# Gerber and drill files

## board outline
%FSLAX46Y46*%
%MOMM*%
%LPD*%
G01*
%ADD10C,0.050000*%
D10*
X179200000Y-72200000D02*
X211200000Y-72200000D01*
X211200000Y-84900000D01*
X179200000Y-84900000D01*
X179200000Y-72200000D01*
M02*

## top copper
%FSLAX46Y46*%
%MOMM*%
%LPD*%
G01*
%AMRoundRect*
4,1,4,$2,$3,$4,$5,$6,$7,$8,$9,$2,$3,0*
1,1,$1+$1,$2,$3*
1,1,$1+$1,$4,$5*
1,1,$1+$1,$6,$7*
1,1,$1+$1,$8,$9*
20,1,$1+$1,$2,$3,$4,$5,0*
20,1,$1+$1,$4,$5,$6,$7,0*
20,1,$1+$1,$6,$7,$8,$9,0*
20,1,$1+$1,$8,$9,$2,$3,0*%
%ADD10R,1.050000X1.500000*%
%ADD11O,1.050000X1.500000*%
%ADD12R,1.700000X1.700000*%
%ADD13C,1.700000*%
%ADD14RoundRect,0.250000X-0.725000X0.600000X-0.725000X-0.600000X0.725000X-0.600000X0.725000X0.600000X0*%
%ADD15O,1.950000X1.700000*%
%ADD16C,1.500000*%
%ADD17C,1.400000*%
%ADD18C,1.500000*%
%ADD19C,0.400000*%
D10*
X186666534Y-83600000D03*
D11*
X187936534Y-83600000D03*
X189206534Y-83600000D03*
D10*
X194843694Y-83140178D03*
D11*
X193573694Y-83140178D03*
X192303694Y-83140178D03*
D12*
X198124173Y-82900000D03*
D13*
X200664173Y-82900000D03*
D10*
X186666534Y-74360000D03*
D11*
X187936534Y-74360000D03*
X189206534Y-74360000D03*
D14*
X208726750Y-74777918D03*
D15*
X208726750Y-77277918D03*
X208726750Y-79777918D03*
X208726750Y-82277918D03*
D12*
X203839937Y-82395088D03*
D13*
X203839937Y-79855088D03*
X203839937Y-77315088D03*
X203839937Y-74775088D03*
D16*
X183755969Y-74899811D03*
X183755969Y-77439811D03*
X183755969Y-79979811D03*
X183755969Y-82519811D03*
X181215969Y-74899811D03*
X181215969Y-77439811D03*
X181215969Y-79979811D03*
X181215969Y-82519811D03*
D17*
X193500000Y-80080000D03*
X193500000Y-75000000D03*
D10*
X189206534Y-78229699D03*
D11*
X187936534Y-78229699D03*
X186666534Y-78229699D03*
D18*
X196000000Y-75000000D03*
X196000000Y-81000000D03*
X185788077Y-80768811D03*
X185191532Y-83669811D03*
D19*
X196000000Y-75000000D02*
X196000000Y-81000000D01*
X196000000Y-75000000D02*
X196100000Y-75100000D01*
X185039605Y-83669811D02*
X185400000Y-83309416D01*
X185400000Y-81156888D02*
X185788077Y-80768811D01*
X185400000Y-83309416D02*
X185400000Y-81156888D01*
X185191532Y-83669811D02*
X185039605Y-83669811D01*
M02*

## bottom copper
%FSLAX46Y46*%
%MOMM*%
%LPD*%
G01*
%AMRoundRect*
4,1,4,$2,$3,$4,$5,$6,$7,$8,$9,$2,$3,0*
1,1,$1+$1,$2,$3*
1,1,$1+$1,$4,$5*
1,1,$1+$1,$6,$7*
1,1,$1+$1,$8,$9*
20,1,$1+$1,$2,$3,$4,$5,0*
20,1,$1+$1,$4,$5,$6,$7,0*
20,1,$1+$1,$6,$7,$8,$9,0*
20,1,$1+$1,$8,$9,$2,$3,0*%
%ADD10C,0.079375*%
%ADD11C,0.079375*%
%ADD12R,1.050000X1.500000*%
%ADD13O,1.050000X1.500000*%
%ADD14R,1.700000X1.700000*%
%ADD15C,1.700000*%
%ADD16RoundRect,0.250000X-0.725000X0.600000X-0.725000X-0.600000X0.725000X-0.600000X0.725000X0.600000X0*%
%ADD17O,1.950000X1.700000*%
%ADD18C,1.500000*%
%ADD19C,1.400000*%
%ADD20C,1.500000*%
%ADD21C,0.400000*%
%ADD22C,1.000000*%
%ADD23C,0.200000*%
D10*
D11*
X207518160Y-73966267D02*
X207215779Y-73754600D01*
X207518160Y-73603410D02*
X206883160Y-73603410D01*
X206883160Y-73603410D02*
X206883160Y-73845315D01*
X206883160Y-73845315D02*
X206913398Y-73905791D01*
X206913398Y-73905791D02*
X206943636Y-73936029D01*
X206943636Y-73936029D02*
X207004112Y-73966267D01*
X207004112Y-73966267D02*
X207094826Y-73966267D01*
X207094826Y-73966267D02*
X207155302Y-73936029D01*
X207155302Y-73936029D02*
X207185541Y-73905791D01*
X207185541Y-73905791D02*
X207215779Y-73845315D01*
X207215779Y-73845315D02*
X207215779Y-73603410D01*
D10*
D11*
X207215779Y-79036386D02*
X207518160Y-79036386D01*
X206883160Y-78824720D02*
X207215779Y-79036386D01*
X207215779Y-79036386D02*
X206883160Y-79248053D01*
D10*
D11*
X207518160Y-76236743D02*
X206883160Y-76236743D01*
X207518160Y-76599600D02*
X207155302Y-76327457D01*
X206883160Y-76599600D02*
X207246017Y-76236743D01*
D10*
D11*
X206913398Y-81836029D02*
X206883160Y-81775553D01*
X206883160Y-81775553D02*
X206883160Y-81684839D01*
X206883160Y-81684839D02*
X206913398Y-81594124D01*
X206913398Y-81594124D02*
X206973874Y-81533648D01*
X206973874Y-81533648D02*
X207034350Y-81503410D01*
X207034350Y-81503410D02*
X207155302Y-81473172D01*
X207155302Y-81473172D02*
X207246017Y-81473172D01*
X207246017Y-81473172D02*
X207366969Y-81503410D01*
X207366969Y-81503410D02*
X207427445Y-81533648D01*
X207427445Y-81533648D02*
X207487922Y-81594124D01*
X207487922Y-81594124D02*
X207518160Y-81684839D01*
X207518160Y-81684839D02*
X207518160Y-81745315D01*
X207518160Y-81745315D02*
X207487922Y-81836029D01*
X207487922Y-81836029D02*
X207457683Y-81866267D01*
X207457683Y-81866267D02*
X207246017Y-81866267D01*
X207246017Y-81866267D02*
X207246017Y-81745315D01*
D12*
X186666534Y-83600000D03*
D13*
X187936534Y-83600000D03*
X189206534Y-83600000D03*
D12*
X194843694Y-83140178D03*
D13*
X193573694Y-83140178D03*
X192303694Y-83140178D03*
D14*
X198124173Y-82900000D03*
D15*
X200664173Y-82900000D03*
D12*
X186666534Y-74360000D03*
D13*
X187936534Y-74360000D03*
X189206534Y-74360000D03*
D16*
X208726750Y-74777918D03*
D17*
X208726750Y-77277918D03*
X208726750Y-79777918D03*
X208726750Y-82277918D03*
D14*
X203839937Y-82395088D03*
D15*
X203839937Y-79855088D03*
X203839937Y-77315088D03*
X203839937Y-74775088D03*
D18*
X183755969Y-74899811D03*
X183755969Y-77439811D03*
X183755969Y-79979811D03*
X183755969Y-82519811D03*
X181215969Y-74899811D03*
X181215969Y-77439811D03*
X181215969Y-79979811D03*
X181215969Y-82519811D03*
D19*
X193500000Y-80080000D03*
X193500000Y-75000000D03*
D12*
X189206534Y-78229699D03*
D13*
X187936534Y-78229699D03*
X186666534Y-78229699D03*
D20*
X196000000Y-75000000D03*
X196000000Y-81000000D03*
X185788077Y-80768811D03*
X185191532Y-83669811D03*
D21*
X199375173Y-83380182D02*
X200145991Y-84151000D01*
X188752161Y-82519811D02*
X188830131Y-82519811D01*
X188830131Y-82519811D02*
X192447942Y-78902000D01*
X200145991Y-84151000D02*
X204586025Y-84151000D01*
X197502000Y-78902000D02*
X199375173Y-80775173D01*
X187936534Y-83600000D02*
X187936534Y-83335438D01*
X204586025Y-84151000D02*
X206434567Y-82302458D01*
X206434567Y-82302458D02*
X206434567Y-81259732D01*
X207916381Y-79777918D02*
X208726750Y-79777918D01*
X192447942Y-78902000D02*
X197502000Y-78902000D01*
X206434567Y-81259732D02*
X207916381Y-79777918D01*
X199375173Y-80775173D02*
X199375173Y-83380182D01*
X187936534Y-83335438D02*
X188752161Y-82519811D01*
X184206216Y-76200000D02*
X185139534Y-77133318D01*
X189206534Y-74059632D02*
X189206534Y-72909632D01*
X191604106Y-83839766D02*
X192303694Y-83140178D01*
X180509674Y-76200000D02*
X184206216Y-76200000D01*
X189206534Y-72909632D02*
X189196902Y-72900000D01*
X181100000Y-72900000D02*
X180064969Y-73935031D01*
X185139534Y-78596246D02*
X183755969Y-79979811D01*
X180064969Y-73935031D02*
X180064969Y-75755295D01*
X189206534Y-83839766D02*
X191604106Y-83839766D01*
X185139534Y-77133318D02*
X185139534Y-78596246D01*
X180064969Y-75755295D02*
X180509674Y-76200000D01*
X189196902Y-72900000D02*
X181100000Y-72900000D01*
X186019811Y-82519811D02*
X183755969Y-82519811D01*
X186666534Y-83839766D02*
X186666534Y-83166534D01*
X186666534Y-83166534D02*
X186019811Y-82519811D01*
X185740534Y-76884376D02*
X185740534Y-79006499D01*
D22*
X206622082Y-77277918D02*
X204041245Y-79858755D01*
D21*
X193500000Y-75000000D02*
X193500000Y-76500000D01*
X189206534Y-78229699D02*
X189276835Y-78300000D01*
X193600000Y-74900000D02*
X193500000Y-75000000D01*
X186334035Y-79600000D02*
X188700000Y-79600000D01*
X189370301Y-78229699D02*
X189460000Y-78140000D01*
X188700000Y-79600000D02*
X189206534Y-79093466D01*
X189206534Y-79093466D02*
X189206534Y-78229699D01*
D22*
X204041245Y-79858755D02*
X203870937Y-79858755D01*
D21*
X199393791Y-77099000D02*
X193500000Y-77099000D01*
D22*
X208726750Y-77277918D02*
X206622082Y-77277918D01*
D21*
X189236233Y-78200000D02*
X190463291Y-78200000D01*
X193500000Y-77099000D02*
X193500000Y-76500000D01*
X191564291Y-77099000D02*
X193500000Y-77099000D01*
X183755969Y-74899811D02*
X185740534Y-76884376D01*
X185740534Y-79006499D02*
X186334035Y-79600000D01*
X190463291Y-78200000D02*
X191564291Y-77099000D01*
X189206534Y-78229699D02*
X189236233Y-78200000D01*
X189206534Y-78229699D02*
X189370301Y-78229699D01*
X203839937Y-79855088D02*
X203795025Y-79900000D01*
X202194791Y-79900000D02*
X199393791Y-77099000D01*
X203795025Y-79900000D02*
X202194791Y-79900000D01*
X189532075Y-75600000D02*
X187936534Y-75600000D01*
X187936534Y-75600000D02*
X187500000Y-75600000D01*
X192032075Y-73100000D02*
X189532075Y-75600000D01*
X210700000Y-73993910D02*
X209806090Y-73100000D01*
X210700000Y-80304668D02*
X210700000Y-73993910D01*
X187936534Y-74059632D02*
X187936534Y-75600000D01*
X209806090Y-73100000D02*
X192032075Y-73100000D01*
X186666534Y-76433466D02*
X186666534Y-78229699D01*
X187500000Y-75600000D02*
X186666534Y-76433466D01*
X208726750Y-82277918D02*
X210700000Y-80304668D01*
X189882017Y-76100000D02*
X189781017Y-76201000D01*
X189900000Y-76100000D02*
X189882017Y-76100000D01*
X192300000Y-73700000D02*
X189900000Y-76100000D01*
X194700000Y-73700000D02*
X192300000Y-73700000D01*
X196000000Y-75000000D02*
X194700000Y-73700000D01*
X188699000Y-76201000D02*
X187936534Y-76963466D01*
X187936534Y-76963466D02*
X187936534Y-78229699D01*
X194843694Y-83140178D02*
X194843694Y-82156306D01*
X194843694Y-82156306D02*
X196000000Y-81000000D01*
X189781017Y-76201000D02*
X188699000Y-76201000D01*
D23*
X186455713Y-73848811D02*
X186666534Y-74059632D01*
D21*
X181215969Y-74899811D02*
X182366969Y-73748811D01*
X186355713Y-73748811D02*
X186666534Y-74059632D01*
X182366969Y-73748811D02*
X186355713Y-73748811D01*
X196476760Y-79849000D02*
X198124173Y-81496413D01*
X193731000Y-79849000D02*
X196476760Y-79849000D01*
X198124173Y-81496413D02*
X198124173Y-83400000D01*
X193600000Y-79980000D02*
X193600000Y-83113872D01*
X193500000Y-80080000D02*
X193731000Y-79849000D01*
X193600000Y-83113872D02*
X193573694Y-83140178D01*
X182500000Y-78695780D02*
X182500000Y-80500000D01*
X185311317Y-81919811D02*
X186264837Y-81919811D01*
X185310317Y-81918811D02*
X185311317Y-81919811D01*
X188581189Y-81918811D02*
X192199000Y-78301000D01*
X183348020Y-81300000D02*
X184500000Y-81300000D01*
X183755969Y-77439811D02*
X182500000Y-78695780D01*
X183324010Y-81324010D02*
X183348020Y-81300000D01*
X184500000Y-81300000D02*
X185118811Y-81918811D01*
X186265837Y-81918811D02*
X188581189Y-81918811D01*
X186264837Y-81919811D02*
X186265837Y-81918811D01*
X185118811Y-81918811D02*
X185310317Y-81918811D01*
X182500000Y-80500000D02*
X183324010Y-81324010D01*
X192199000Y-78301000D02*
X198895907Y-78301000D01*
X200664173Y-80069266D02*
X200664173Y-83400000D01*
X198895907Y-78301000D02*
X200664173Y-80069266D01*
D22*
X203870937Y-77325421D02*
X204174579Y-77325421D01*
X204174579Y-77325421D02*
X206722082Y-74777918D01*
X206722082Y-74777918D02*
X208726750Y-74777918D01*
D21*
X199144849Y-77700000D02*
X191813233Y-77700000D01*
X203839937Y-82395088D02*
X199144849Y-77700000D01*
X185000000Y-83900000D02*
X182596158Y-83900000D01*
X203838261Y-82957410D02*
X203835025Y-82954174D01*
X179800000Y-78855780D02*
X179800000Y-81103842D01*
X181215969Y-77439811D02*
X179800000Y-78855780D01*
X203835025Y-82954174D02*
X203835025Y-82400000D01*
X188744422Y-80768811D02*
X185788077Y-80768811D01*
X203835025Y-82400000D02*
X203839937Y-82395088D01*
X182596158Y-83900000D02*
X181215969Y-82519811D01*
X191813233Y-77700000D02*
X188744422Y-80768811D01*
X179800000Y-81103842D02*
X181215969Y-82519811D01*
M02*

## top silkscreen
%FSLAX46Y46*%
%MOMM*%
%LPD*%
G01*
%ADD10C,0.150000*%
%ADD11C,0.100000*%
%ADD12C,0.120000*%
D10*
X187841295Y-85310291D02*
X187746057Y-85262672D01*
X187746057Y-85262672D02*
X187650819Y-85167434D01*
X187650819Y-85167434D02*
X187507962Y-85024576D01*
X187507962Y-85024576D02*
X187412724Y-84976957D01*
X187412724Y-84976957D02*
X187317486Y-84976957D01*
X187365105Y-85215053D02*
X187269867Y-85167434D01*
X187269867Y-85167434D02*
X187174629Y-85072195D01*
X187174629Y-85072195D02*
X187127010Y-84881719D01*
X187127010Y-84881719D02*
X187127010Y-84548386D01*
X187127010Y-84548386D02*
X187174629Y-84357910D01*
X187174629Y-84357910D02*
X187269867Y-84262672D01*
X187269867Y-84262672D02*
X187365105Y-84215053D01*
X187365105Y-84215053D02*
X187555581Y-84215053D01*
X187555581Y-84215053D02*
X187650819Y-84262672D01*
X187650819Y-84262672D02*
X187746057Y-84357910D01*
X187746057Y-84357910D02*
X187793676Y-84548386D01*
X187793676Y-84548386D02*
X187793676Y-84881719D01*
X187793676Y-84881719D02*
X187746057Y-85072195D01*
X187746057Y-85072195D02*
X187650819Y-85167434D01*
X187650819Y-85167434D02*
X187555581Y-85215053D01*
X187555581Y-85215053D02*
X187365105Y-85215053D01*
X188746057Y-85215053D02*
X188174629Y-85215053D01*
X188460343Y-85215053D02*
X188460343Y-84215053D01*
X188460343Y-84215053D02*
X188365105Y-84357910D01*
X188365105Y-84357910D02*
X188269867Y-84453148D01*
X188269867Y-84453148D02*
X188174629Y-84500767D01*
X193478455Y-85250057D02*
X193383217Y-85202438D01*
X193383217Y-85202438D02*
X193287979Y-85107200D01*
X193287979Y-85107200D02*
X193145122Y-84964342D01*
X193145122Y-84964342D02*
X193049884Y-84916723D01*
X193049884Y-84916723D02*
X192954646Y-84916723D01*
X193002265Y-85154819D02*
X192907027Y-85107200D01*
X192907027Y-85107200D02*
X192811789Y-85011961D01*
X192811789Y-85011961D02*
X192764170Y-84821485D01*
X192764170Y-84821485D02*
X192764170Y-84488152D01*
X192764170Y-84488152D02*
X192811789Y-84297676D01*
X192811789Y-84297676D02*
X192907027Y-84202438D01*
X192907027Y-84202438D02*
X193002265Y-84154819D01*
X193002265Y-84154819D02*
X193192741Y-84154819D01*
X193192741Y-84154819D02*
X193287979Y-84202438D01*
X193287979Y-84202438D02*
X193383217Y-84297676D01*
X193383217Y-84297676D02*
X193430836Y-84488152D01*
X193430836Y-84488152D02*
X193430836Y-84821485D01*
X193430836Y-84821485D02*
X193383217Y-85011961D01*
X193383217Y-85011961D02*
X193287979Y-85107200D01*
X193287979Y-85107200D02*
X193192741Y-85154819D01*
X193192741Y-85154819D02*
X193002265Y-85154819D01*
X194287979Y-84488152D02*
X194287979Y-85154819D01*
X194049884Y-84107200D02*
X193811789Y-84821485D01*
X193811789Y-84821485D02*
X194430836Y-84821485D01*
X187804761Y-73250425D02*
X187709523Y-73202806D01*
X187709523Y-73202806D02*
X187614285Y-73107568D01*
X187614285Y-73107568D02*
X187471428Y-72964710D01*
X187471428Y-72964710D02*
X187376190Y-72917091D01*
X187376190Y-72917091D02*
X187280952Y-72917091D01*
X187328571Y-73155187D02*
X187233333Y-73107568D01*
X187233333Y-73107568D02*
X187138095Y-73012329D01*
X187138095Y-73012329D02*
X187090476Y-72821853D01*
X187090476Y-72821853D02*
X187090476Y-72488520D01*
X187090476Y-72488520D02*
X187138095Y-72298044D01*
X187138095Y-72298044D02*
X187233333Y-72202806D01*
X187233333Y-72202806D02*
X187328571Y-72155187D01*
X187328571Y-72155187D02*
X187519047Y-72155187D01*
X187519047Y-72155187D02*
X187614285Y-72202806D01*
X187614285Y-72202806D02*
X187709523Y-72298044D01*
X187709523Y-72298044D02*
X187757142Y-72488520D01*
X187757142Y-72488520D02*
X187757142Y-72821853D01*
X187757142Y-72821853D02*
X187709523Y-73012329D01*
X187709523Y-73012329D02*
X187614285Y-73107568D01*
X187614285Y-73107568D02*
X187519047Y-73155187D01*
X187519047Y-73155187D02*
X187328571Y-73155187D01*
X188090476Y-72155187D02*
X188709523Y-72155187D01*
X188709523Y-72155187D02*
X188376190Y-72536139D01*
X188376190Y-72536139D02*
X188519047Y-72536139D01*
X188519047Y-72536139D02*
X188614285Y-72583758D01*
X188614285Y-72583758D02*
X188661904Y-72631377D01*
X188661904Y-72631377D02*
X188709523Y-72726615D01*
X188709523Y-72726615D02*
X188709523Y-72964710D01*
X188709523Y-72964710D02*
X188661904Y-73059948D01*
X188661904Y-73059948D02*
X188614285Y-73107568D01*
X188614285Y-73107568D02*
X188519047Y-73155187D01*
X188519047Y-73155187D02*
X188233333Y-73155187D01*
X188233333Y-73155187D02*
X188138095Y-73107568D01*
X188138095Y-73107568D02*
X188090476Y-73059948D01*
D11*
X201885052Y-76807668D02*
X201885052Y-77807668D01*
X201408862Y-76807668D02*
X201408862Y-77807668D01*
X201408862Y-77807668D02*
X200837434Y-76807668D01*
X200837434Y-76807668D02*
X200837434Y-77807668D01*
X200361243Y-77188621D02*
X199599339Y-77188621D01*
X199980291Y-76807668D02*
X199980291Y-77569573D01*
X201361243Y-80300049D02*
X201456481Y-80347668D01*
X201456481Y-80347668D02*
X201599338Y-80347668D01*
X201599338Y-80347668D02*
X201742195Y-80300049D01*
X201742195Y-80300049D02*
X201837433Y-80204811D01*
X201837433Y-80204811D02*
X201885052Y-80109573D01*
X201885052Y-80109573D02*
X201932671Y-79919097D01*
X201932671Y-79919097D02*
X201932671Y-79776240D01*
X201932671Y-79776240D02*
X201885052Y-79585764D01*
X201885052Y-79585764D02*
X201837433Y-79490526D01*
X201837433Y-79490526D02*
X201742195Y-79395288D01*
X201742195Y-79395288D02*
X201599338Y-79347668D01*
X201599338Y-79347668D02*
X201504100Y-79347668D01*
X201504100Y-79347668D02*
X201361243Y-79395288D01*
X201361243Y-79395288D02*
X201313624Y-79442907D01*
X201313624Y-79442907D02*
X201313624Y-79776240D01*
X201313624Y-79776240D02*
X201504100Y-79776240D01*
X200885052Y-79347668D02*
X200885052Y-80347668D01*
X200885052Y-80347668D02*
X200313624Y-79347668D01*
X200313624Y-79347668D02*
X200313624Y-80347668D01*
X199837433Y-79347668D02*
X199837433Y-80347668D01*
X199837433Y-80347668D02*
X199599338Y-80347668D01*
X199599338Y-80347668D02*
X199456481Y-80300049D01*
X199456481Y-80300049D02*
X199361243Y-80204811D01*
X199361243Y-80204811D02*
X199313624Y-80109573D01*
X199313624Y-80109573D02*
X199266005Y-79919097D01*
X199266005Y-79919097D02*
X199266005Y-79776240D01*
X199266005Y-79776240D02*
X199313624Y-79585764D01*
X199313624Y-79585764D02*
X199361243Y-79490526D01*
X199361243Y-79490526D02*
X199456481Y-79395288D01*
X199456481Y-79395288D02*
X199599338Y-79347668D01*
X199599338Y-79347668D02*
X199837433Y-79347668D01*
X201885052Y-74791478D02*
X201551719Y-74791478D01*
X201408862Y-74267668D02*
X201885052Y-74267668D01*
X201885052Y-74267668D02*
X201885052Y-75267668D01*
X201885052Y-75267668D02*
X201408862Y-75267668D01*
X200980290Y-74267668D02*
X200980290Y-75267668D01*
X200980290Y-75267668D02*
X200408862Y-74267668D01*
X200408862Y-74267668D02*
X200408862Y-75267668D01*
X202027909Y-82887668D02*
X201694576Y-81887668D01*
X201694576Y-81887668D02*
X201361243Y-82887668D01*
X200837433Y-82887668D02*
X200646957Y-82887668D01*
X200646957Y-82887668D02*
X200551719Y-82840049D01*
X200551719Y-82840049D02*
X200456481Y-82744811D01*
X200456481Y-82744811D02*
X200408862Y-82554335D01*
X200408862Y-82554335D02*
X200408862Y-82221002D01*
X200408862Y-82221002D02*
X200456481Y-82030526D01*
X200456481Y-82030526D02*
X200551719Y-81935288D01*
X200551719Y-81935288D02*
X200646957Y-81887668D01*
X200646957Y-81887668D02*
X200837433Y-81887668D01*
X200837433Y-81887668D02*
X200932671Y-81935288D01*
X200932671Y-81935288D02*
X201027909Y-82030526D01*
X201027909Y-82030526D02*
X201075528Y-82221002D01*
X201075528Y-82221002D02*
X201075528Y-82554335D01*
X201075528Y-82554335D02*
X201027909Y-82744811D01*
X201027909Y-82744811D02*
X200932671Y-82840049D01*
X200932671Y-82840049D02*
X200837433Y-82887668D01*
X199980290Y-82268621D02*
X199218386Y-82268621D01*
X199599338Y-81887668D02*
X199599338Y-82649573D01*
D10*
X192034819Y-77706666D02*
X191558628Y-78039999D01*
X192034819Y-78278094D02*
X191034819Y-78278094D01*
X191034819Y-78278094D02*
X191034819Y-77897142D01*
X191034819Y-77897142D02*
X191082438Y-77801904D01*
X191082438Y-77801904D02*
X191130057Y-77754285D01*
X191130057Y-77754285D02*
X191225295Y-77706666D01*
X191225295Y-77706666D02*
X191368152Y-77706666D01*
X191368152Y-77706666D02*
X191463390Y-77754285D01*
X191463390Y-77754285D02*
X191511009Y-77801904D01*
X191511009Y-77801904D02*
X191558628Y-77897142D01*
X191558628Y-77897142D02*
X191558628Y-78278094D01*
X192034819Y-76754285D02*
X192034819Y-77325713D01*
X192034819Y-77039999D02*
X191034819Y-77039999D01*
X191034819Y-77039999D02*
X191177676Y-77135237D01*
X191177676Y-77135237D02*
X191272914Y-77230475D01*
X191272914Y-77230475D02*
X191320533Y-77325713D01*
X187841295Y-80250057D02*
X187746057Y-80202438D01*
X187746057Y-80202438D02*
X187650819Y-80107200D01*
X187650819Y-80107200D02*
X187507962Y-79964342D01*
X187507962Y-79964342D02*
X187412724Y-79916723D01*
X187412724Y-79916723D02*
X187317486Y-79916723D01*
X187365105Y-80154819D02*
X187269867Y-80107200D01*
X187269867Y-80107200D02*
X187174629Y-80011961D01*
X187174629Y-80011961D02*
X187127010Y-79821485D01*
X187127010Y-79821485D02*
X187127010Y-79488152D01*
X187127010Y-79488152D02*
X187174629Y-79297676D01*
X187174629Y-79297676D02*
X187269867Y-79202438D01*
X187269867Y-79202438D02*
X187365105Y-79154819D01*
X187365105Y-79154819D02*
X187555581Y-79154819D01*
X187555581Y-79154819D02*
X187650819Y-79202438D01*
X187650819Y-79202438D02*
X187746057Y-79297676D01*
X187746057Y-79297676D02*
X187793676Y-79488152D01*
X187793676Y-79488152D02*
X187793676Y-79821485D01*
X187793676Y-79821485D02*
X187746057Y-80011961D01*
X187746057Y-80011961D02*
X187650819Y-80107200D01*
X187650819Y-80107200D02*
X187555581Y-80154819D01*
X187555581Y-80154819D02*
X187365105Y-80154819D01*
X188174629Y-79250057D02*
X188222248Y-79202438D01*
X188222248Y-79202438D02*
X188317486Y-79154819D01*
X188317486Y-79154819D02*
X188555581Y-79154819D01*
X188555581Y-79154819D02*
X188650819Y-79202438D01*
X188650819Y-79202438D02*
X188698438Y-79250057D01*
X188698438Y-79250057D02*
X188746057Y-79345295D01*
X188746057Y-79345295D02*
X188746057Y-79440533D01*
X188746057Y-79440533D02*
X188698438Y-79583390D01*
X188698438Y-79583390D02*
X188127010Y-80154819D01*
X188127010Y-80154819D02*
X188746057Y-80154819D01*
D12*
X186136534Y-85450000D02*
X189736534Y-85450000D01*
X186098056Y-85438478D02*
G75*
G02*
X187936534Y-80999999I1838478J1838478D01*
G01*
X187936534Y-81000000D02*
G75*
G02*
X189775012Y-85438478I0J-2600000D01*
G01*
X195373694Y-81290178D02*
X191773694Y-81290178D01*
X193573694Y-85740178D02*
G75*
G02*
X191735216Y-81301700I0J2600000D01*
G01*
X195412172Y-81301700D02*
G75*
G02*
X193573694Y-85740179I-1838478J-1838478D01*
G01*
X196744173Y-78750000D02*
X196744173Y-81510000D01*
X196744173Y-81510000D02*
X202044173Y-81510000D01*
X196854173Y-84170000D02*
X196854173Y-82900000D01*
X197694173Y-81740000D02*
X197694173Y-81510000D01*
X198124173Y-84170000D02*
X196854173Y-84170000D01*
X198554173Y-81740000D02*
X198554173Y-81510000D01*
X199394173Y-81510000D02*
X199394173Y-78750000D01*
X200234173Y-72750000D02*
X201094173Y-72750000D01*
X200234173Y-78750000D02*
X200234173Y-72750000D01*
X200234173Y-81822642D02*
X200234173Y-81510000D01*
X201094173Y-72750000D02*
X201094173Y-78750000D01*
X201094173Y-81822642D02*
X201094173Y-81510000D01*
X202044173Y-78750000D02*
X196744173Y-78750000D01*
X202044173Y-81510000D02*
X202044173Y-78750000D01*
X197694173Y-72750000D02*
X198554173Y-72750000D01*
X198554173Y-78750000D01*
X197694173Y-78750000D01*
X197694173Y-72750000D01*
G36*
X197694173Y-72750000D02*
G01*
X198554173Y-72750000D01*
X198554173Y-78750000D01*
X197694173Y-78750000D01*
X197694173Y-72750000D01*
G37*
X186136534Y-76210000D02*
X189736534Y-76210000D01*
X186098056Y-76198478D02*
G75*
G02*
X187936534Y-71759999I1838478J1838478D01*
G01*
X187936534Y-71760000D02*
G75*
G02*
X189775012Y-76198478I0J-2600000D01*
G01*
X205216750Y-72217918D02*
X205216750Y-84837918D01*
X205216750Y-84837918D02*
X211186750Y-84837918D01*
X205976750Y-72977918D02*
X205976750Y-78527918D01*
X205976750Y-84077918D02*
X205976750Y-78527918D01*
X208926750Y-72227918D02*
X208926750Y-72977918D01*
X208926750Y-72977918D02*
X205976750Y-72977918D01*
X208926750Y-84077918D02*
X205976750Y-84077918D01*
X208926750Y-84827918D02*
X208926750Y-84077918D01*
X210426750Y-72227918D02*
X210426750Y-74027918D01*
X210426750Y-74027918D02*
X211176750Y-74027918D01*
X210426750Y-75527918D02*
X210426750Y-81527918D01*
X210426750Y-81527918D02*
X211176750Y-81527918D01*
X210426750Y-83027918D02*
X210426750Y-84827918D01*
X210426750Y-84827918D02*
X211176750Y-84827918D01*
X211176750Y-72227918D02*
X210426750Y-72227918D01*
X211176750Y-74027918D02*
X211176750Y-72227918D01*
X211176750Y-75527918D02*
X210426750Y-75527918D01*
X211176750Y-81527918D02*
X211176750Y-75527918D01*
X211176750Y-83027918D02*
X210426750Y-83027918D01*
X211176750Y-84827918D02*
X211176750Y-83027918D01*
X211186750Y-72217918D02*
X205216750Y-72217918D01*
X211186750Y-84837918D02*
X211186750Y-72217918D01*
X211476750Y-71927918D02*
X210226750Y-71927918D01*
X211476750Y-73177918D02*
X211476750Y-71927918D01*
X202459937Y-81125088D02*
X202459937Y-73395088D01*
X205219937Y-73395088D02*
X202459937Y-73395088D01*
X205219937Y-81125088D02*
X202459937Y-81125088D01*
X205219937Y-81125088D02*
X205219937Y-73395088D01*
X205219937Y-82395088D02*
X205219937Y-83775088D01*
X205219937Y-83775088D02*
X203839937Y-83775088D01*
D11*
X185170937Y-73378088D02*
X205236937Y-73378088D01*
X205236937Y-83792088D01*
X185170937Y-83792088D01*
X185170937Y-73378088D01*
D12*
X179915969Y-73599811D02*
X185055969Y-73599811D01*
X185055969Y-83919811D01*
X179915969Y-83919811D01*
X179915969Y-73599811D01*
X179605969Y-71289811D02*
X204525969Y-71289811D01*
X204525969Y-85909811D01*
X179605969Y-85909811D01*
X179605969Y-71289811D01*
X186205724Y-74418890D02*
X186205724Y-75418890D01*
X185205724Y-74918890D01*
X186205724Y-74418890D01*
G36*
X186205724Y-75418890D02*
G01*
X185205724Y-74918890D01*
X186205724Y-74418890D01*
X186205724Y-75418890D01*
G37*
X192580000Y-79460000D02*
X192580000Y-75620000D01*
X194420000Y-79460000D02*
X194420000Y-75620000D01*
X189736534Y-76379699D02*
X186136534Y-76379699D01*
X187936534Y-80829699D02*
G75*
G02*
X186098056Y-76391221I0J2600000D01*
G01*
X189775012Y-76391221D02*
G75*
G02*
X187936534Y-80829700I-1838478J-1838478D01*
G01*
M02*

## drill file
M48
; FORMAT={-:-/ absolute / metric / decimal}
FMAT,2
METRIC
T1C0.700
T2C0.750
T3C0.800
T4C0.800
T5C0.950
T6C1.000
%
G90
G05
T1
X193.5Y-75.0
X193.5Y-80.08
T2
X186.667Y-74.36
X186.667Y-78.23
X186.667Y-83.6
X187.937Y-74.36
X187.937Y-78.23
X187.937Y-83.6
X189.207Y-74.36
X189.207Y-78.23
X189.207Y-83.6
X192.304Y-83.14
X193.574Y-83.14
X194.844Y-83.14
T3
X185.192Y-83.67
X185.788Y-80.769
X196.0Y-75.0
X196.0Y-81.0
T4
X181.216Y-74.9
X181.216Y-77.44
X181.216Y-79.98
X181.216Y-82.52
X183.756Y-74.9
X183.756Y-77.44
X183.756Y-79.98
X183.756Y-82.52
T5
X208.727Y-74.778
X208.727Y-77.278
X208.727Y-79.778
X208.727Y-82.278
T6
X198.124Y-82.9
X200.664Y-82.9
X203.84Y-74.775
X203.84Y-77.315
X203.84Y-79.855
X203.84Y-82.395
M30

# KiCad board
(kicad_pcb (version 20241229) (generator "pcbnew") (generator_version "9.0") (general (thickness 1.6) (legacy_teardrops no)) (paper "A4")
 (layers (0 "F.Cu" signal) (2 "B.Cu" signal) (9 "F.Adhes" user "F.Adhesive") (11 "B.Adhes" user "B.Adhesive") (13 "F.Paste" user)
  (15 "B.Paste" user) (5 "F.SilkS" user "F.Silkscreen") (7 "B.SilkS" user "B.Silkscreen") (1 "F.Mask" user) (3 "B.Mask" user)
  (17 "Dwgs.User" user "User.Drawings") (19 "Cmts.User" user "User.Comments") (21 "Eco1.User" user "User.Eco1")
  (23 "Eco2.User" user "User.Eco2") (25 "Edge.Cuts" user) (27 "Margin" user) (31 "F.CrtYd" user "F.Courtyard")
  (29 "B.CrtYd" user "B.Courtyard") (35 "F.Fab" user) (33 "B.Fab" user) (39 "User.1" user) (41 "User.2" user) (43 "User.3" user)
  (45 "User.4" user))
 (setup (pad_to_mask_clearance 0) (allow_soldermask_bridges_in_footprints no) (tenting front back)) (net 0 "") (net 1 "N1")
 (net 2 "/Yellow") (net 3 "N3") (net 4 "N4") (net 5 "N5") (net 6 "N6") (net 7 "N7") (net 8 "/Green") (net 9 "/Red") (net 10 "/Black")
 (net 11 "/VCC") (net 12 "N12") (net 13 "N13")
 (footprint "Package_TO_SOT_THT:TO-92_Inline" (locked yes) (layer "F.Cu") (at 186.666534 83.6)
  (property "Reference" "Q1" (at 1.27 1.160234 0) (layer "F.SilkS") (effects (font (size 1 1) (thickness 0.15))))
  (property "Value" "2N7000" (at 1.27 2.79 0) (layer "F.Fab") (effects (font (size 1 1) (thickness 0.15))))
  (fp_line (start -0.53 1.85) (end 3.07 1.85) (stroke (width 0.12) (type solid)) (layer "F.SilkS"))
  (fp_arc (start -0.568478 1.838478) (mid -1.132087 -0.994977) (end 1.27 -2.6) (stroke (width 0.12) (type solid)) (layer "F.SilkS"))
  (fp_arc (start 1.27 -2.6) (mid 3.672087 -0.994977) (end 3.108478 1.838478) (stroke (width 0.12) (type solid)) (layer "F.SilkS"))
  (pad "1" thru_hole rect (at 0 0) (size 1.05 1.5) (drill 0.75) (layers "*.Cu" "*.Mask") (remove_unused_layers no) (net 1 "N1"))
  (pad "2" thru_hole oval (at 1.27 0) (size 1.05 1.5) (drill 0.75) (layers "*.Cu" "*.Mask") (remove_unused_layers no) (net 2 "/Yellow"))
  (pad "3" thru_hole oval (at 2.54 0) (size 1.05 1.5) (drill 0.75) (layers "*.Cu" "*.Mask") (remove_unused_layers no) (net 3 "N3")))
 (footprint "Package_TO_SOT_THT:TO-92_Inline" (layer "F.Cu") (at 194.843694 83.140178 180)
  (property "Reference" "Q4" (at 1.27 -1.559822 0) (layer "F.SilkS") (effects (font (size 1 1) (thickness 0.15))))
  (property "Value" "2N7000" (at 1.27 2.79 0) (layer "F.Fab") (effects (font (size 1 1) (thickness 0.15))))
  (fp_line (start -0.53 1.85) (end 3.07 1.85) (stroke (width 0.12) (type solid)) (layer "F.SilkS"))
  (fp_arc (start 1.27 -2.6) (mid 3.672087 -0.994977) (end 3.108478 1.838478) (stroke (width 0.12) (type solid)) (layer "F.SilkS"))
  (fp_arc (start -0.568478 1.838478) (mid -1.132087 -0.994977) (end 1.27 -2.6) (stroke (width 0.12) (type solid)) (layer "F.SilkS"))
  (pad "1" thru_hole rect (at 0 0 180) (size 1.05 1.5) (drill 0.75) (layers "*.Cu" "*.Mask") (remove_unused_layers no) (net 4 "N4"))
  (pad "2" thru_hole oval (at 1.27 0 180) (size 1.05 1.5) (drill 0.75) (layers "*.Cu" "*.Mask") (remove_unused_layers no) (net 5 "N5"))
  (pad "3" thru_hole oval (at 2.54 0 180) (size 1.05 1.5) (drill 0.75) (layers "*.Cu" "*.Mask") (remove_unused_layers no) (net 3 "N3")))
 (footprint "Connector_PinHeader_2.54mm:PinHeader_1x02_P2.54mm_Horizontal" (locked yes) (layer "F.Cu") (at 198.124173 82.9 90)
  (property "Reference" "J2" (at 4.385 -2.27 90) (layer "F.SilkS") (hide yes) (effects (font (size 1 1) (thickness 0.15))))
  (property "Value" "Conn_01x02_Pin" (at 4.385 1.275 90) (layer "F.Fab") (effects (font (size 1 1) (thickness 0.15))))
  (fp_line (start 4.15 -1.38) (end 1.39 -1.38) (stroke (width 0.12) (type solid)) (layer "F.SilkS"))
  (fp_line (start 1.39 -1.38) (end 1.39 3.92) (stroke (width 0.12) (type solid)) (layer "F.SilkS"))
  (fp_line (start -1.27 -1.27) (end 0 -1.27) (stroke (width 0.12) (type solid)) (layer "F.SilkS"))
  (fp_line (start 1.16 -0.43) (end 1.39 -0.43) (stroke (width 0.12) (type solid)) (layer "F.SilkS"))
  (fp_line (start -1.27 0) (end -1.27 -1.27) (stroke (width 0.12) (type solid)) (layer "F.SilkS"))
  (fp_line (start 1.16 0.43) (end 1.39 0.43) (stroke (width 0.12) (type solid)) (layer "F.SilkS"))
  (fp_line (start 1.39 1.27) (end 4.15 1.27) (stroke (width 0.12) (type solid)) (layer "F.SilkS"))
  (fp_line (start 10.15 2.11) (end 10.15 2.97) (stroke (width 0.12) (type solid)) (layer "F.SilkS"))
  (fp_line (start 4.15 2.11) (end 10.15 2.11) (stroke (width 0.12) (type solid)) (layer "F.SilkS"))
  (fp_line (start 1.077358 2.11) (end 1.39 2.11) (stroke (width 0.12) (type solid)) (layer "F.SilkS"))
  (fp_line (start 10.15 2.97) (end 4.15 2.97) (stroke (width 0.12) (type solid)) (layer "F.SilkS"))
  (fp_line (start 1.077358 2.97) (end 1.39 2.97) (stroke (width 0.12) (type solid)) (layer "F.SilkS"))
  (fp_line (start 4.15 3.92) (end 4.15 -1.38) (stroke (width 0.12) (type solid)) (layer "F.SilkS"))
  (fp_line (start 1.39 3.92) (end 4.15 3.92) (stroke (width 0.12) (type solid)) (layer "F.SilkS"))
  (fp_rect (start 4.15 -0.43) (end 10.15 0.43) (stroke (width 0.12) (type solid)) (fill yes) (layer "F.SilkS"))
  (pad "1" thru_hole rect (at 0 0 90) (size 1.7 1.7) (drill 1) (layers "*.Cu" "*.Mask") (remove_unused_layers no) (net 5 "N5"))
  (pad "2" thru_hole circle (at 0 2.54 90) (size 1.7 1.7) (drill 1) (layers "*.Cu" "*.Mask") (remove_unused_layers no) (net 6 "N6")))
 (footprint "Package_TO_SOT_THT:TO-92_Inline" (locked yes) (layer "F.Cu") (at 186.666534 74.36)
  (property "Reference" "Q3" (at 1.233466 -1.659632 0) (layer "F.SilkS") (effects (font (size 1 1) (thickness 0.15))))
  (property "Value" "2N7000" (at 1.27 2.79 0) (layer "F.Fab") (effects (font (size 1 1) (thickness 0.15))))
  (fp_line (start -0.53 1.85) (end 3.07 1.85) (stroke (width 0.12) (type solid)) (layer "F.SilkS"))
  (fp_arc (start -0.568478 1.838478) (mid -1.132087 -0.994977) (end 1.27 -2.6) (stroke (width 0.12) (type solid)) (layer "F.SilkS"))
  (fp_arc (start 1.27 -2.6) (mid 3.672087 -0.994977) (end 3.108478 1.838478) (stroke (width 0.12) (type solid)) (layer "F.SilkS"))
  (pad "1" thru_hole rect (at 0 0) (size 1.05 1.5) (drill 0.75) (layers "*.Cu" "*.Mask") (remove_unused_layers no) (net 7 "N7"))
  (pad "2" thru_hole oval (at 1.27 0) (size 1.05 1.5) (drill 0.75) (layers "*.Cu" "*.Mask") (remove_unused_layers no) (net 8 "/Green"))
  (pad "3" thru_hole oval (at 2.54 0) (size 1.05 1.5) (drill 0.75) (layers "*.Cu" "*.Mask") (remove_unused_layers no) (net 3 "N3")))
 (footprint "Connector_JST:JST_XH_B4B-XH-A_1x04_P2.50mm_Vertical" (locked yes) (layer "F.Cu") (at 208.72675 74.777918 -90)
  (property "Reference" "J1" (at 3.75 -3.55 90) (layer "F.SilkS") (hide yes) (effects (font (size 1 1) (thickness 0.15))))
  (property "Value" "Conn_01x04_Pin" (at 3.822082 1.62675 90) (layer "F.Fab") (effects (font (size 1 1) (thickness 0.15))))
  (fp_line (start -2.56 3.51) (end 10.06 3.51) (stroke (width 0.12) (type solid)) (layer "F.SilkS"))
  (fp_line (start 10.06 3.51) (end 10.06 -2.46) (stroke (width 0.12) (type solid)) (layer "F.SilkS"))
  (fp_line (start -1.8 2.75) (end 3.75 2.75) (stroke (width 0.12) (type solid)) (layer "F.SilkS"))
  (fp_line (start 9.3 2.75) (end 3.75 2.75) (stroke (width 0.12) (type solid)) (layer "F.SilkS"))
  (fp_line (start -2.55 -0.2) (end -1.8 -0.2) (stroke (width 0.12) (type solid)) (layer "F.SilkS"))
  (fp_line (start -1.8 -0.2) (end -1.8 2.75) (stroke (width 0.12) (type solid)) (layer "F.SilkS"))
  (fp_line (start 9.3 -0.2) (end 9.3 2.75) (stroke (width 0.12) (type solid)) (layer "F.SilkS"))
  (fp_line (start 10.05 -0.2) (end 9.3 -0.2) (stroke (width 0.12) (type solid)) (layer "F.SilkS"))
  (fp_line (start -2.55 -1.7) (end -0.75 -1.7) (stroke (width 0.12) (type solid)) (layer "F.SilkS"))
  (fp_line (start -0.75 -1.7) (end -0.75 -2.45) (stroke (width 0.12) (type solid)) (layer "F.SilkS"))
  (fp_line (start 0.75 -1.7) (end 6.75 -1.7) (stroke (width 0.12) (type solid)) (layer "F.SilkS"))
  (fp_line (start 6.75 -1.7) (end 6.75 -2.45) (stroke (width 0.12) (type solid)) (layer "F.SilkS"))
  (fp_line (start 8.25 -1.7) (end 10.05 -1.7) (stroke (width 0.12) (type solid)) (layer "F.SilkS"))
  (fp_line (start 10.05 -1.7) (end 10.05 -2.45) (stroke (width 0.12) (type solid)) (layer "F.SilkS"))
  (fp_line (start -2.55 -2.45) (end -2.55 -1.7) (stroke (width 0.12) (type solid)) (layer "F.SilkS"))
  (fp_line (start -0.75 -2.45) (end -2.55 -2.45) (stroke (width 0.12) (type solid)) (layer "F.SilkS"))
  (fp_line (start 0.75 -2.45) (end 0.75 -1.7) (stroke (width 0.12) (type solid)) (layer "F.SilkS"))
  (fp_line (start 6.75 -2.45) (end 0.75 -2.45) (stroke (width 0.12) (type solid)) (layer "F.SilkS"))
  (fp_line (start 8.25 -2.45) (end 8.25 -1.7) (stroke (width 0.12) (type solid)) (layer "F.SilkS"))
  (fp_line (start 10.05 -2.45) (end 8.25 -2.45) (stroke (width 0.12) (type solid)) (layer "F.SilkS"))
  (fp_line (start -2.56 -2.46) (end -2.56 3.51) (stroke (width 0.12) (type solid)) (layer "F.SilkS"))
  (fp_line (start 10.06 -2.46) (end -2.56 -2.46) (stroke (width 0.12) (type solid)) (layer "F.SilkS"))
  (fp_line (start -2.85 -2.75) (end -2.85 -1.5) (stroke (width 0.12) (type solid)) (layer "F.SilkS"))
  (fp_line (start -1.6 -2.75) (end -2.85 -2.75) (stroke (width 0.12) (type solid)) (layer "F.SilkS"))
  (pad "1" thru_hole roundrect (at 0 0 270) (size 1.7 1.95) (drill 0.95) (layers "*.Cu" "*.Mask") (remove_unused_layers no)
   (roundrect_rratio 0.147059) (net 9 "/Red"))
  (pad "2" thru_hole oval (at 2.5 0 270) (size 1.7 1.95) (drill 0.95) (layers "*.Cu" "*.Mask") (remove_unused_layers no) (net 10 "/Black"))
  (pad "3" thru_hole oval (at 5 0 270) (size 1.7 1.95) (drill 0.95) (layers "*.Cu" "*.Mask") (remove_unused_layers no) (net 2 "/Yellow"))
  (pad "4" thru_hole oval (at 7.5 0 270) (size 1.7 1.95) (drill 0.95) (layers "*.Cu" "*.Mask") (remove_unused_layers no) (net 8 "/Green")))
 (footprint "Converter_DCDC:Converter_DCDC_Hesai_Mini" (layer "F.Cu") (at 185.170937 83.792088 90)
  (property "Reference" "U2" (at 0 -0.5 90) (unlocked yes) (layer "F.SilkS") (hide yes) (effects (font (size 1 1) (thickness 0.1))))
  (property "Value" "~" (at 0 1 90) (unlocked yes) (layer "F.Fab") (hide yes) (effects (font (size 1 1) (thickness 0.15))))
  (fp_line (start 2.667 17.289) (end 10.397 17.289) (stroke (width 0.12) (type solid)) (layer "F.SilkS"))
  (fp_line (start 10.397 20.049) (end 10.397 17.289) (stroke (width 0.12) (type solid)) (layer "F.SilkS"))
  (fp_line (start 2.667 20.049) (end 2.667 17.289) (stroke (width 0.12) (type solid)) (layer "F.SilkS"))
  (fp_line (start 2.667 20.049) (end 10.397 20.049) (stroke (width 0.12) (type solid)) (layer "F.SilkS"))
  (fp_line (start 1.397 20.049) (end 0.017 20.049) (stroke (width 0.12) (type solid)) (layer "F.SilkS"))
  (fp_line (start 0.017 20.049) (end 0.017 18.669) (stroke (width 0.12) (type solid)) (layer "F.SilkS"))
  (fp_rect (start 0 0) (end 10.414 20.066) (stroke (width 0.1) (type default)) (fill no) (layer "F.SilkS"))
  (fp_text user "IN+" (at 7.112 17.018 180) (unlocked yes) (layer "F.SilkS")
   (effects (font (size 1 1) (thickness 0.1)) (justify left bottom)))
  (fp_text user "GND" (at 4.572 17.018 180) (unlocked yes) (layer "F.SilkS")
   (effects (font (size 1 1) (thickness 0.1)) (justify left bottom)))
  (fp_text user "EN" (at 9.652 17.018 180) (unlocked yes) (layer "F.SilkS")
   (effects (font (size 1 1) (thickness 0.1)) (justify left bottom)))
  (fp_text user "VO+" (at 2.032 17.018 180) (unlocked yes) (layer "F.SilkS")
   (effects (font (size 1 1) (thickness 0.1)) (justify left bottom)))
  (pad "1" thru_hole rect (at 1.397 18.669 180) (size 1.7 1.7) (drill 1) (layers "*.Cu" "*.Mask") (remove_unused_layers no) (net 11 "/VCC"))
  (pad "2" thru_hole circle (at 3.937 18.669 180) (size 1.7 1.7) (drill 1) (layers "*.Cu" "*.Mask") (remove_unused_layers no)
   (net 10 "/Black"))
  (pad "3" thru_hole circle (at 6.477 18.669 180) (size 1.7 1.7) (drill 1) (layers "*.Cu" "*.Mask") (remove_unused_layers no) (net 9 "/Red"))
  (pad "4" thru_hole circle (at 9.017 18.669 180) (size 1.7 1.7) (drill 1) (layers "*.Cu" "*.Mask") (remove_unused_layers no) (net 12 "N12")))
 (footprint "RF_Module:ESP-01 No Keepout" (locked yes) (layer "F.Cu") (at 183.755969 74.899811 -90)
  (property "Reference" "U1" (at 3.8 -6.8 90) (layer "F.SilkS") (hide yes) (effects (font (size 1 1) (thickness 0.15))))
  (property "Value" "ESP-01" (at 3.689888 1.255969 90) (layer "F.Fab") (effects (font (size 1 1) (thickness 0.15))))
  (fp_rect (start -1.3 -1.3) (end 9.02 3.84) (stroke (width 0.12) (type default)) (fill no) (layer "F.SilkS"))
  (fp_rect (start -3.61 -20.77) (end 11.01 4.15) (stroke (width 0.12) (type default)) (fill no) (layer "F.SilkS"))
  (fp_poly
   (pts (xy -0.480921 -2.449755) (xy 0.519079 -2.449755) (xy 0.019079 -1.449755)) (stroke (width 0.12) (type solid)) (fill yes)
   (layer "F.SilkS"))
  (pad "1" thru_hole circle (at 0 0 270) (size 1.5 1.5) (drill 0.8) (layers "*.Cu" "*.Mask") (remove_unused_layers no) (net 10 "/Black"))
  (pad "2" thru_hole circle (at 2.54 0 270) (size 1.5 1.5) (drill 0.8) (layers "*.Cu" "*.Mask") (remove_unused_layers no) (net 6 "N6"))
  (pad "3" thru_hole circle (at 5.08 0 270) (size 1.5 1.5) (drill 0.8) (layers "*.Cu" "*.Mask") (remove_unused_layers no) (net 3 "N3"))
  (pad "4" thru_hole circle (at 7.62 0 270) (size 1.5 1.5) (drill 0.8) (layers "*.Cu" "*.Mask") (remove_unused_layers no) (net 1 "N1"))
  (pad "5" thru_hole circle (at 0 2.54 270) (size 1.5 1.5) (drill 0.8) (layers "*.Cu" "*.Mask") (remove_unused_layers no) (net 7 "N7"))
  (pad "6" thru_hole circle (at 2.54 2.54 270) (size 1.5 1.5) (drill 0.8) (layers "*.Cu" "*.Mask") (remove_unused_layers no) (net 11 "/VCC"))
  (pad "7" thru_hole circle (at 5.08 2.54 270) (size 1.5 1.5) (drill 0.8) (layers "*.Cu" "*.Mask") (remove_unused_layers no) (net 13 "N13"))
  (pad "8" thru_hole circle (at 7.62 2.54 270) (size 1.5 1.5) (drill 0.8) (layers "*.Cu" "*.Mask") (remove_unused_layers no) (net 11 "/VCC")))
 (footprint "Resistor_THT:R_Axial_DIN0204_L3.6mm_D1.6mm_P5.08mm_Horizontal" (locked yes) (layer "F.Cu") (at 193.5 80.08 90)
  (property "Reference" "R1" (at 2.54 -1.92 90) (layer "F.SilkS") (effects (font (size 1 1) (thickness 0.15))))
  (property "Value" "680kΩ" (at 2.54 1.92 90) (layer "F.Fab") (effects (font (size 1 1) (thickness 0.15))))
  (fp_line (start 0.62 -0.92) (end 4.46 -0.92) (stroke (width 0.12) (type solid)) (layer "F.SilkS"))
  (fp_line (start 0.62 0.92) (end 4.46 0.92) (stroke (width 0.12) (type solid)) (layer "F.SilkS"))
  (pad "1" thru_hole circle (at 0 0 90) (size 1.4 1.4) (drill 0.7) (layers "*.Cu" "*.Mask") (remove_unused_layers no) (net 5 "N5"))
  (pad "2" thru_hole circle (at 5.08 0 90) (size 1.4 1.4) (drill 0.7) (layers "*.Cu" "*.Mask") (remove_unused_layers no) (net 10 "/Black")))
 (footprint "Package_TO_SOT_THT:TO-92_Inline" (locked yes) (layer "F.Cu") (at 189.206534 78.229699 180)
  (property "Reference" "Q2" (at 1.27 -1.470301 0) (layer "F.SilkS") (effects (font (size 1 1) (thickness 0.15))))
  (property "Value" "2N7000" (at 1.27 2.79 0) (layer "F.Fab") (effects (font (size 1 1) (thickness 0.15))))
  (fp_line (start -0.53 1.85) (end 3.07 1.85) (stroke (width 0.12) (type solid)) (layer "F.SilkS"))
  (fp_arc (start 1.27 -2.6) (mid 3.672087 -0.994977) (end 3.108478 1.838478) (stroke (width 0.12) (type solid)) (layer "F.SilkS"))
  (fp_arc (start -0.568478 1.838478) (mid -1.132087 -0.994977) (end 1.27 -2.6) (stroke (width 0.12) (type solid)) (layer "F.SilkS"))
  (pad "1" thru_hole rect (at 0 0 180) (size 1.05 1.5) (drill 0.75) (layers "*.Cu" "*.Mask") (remove_unused_layers no) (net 10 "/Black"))
  (pad "2" thru_hole oval (at 1.27 0 180) (size 1.05 1.5) (drill 0.75) (layers "*.Cu" "*.Mask") (remove_unused_layers no) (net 4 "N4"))
  (pad "3" thru_hole oval (at 2.54 0 180) (size 1.05 1.5) (drill 0.75) (layers "*.Cu" "*.Mask") (remove_unused_layers no) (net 8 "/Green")))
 (gr_rect (start 179.2 72.2) (end 211.2 84.9) (stroke (width 0.05) (type default)) (fill no) (layer "Edge.Cuts"))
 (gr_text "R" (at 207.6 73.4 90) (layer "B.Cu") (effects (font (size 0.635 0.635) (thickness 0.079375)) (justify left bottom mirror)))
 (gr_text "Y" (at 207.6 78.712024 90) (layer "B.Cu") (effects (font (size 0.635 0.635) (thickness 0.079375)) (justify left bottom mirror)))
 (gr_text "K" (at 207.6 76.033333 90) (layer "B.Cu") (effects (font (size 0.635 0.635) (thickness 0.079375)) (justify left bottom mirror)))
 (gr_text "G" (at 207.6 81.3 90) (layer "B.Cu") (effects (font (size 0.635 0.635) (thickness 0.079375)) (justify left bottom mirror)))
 (segment (start 199.375173 83.380182) (end 200.145991 84.151) (width 0.4) (layer "B.Cu") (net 2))
 (segment (start 188.752161 82.519811) (end 188.830131 82.519811) (width 0.4) (layer "B.Cu") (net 2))
 (segment (start 188.830131 82.519811) (end 192.447942 78.902) (width 0.4) (layer "B.Cu") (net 2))
 (segment (start 200.145991 84.151) (end 204.586025 84.151) (width 0.4) (layer "B.Cu") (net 2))
 (segment (start 197.502 78.902) (end 199.375173 80.775173) (width 0.4) (layer "B.Cu") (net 2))
 (segment (start 187.936534 83.6) (end 187.936534 83.335438) (width 0.4) (layer "B.Cu") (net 2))
 (segment (start 204.586025 84.151) (end 206.434567 82.302458) (width 0.4) (layer "B.Cu") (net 2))
 (segment (start 206.434567 82.302458) (end 206.434567 81.259732) (width 0.4) (layer "B.Cu") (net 2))
 (segment (start 207.916381 79.777918) (end 208.72675 79.777918) (width 0.4) (layer "B.Cu") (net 2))
 (segment (start 192.447942 78.902) (end 197.502 78.902) (width 0.4) (layer "B.Cu") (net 2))
 (segment (start 206.434567 81.259732) (end 207.916381 79.777918) (width 0.4) (layer "B.Cu") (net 2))
 (segment (start 199.375173 80.775173) (end 199.375173 83.380182) (width 0.4) (layer "B.Cu") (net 2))
 (segment (start 187.936534 83.335438) (end 188.752161 82.519811) (width 0.4) (layer "B.Cu") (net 2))
 (segment (start 184.206216 76.2) (end 185.139534 77.133318) (width 0.4) (layer "B.Cu") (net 3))
 (segment (start 189.206534 74.059632) (end 189.206534 72.909632) (width 0.4) (layer "B.Cu") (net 3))
 (segment (start 191.604106 83.839766) (end 192.303694 83.140178) (width 0.4) (layer "B.Cu") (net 3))
 (segment (start 180.509674 76.2) (end 184.206216 76.2) (width 0.4) (layer "B.Cu") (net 3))
 (segment (start 189.206534 72.909632) (end 189.196902 72.9) (width 0.4) (layer "B.Cu") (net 3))
 (segment (start 181.1 72.9) (end 180.064969 73.935031) (width 0.4) (layer "B.Cu") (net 3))
 (segment (start 185.139534 78.596246) (end 183.755969 79.979811) (width 0.4) (layer "B.Cu") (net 3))
 (segment (start 180.064969 73.935031) (end 180.064969 75.755295) (width 0.4) (layer "B.Cu") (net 3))
 (segment (start 189.206534 83.839766) (end 191.604106 83.839766) (width 0.4) (layer "B.Cu") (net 3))
 (segment (start 185.139534 77.133318) (end 185.139534 78.596246) (width 0.4) (layer "B.Cu") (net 3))
 (segment (start 180.064969 75.755295) (end 180.509674 76.2) (width 0.4) (layer "B.Cu") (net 3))
 (segment (start 189.196902 72.9) (end 181.1 72.9) (width 0.4) (layer "B.Cu") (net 3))
 (segment (start 186.019811 82.519811) (end 183.755969 82.519811) (width 0.4) (layer "B.Cu") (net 1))
 (segment (start 186.666534 83.839766) (end 186.666534 83.166534) (width 0.4) (layer "B.Cu") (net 1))
 (segment (start 186.666534 83.166534) (end 186.019811 82.519811) (width 0.4) (layer "B.Cu") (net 1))
 (segment (start 185.740534 76.884376) (end 185.740534 79.006499) (width 0.4) (layer "B.Cu") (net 10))
 (segment (start 206.622082 77.277918) (end 204.041245 79.858755) (width 1) (layer "B.Cu") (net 10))
 (segment (start 193.5 75) (end 193.5 76.5) (width 0.4) (layer "B.Cu") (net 10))
 (segment (start 189.206534 78.229699) (end 189.276835 78.3) (width 0.4) (layer "B.Cu") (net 10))
 (segment (start 193.6 74.9) (end 193.5 75) (width 0.4) (layer "B.Cu") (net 10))
 (segment (start 186.334035 79.6) (end 188.7 79.6) (width 0.4) (layer "B.Cu") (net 10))
 (segment (start 189.370301 78.229699) (end 189.46 78.14) (width 0.4) (layer "B.Cu") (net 10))
 (segment (start 188.7 79.6) (end 189.206534 79.093466) (width 0.4) (layer "B.Cu") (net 10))
 (segment (start 189.206534 79.093466) (end 189.206534 78.229699) (width 0.4) (layer "B.Cu") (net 10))
 (segment (start 204.041245 79.858755) (end 203.870937 79.858755) (width 1) (layer "B.Cu") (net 10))
 (segment (start 199.393791 77.099) (end 193.5 77.099) (width 0.4) (layer "B.Cu") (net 10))
 (segment (start 208.72675 77.277918) (end 206.622082 77.277918) (width 1) (layer "B.Cu") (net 10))
 (segment (start 189.236233 78.2) (end 190.463291 78.2) (width 0.4) (layer "B.Cu") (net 10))
 (segment (start 193.5 77.099) (end 193.5 76.5) (width 0.4) (layer "B.Cu") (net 10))
 (segment (start 191.564291 77.099) (end 193.5 77.099) (width 0.4) (layer "B.Cu") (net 10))
 (segment (start 183.755969 74.899811) (end 185.740534 76.884376) (width 0.4) (layer "B.Cu") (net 10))
 (segment (start 185.740534 79.006499) (end 186.334035 79.6) (width 0.4) (layer "B.Cu") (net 10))
 (segment (start 190.463291 78.2) (end 191.564291 77.099) (width 0.4) (layer "B.Cu") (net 10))
 (segment (start 189.206534 78.229699) (end 189.236233 78.2) (width 0.4) (layer "B.Cu") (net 10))
 (segment (start 189.206534 78.229699) (end 189.370301 78.229699) (width 0.4) (layer "B.Cu") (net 10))
 (segment (start 203.839937 79.855088) (end 203.795025 79.9) (width 0.4) (layer "B.Cu") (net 10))
 (segment (start 202.194791 79.9) (end 199.393791 77.099) (width 0.4) (layer "B.Cu") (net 10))
 (segment (start 203.795025 79.9) (end 202.194791 79.9) (width 0.4) (layer "B.Cu") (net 10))
 (segment (start 189.532075 75.6) (end 187.936534 75.6) (width 0.4) (layer "B.Cu") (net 8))
 (segment (start 187.936534 75.6) (end 187.5 75.6) (width 0.4) (layer "B.Cu") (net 8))
 (segment (start 192.032075 73.1) (end 189.532075 75.6) (width 0.4) (layer "B.Cu") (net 8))
 (segment (start 210.7 73.99391) (end 209.80609 73.1) (width 0.4) (layer "B.Cu") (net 8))
 (segment (start 210.7 80.304668) (end 210.7 73.99391) (width 0.4) (layer "B.Cu") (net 8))
 (segment (start 187.936534 74.059632) (end 187.936534 75.6) (width 0.4) (layer "B.Cu") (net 8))
 (segment (start 209.80609 73.1) (end 192.032075 73.1) (width 0.4) (layer "B.Cu") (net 8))
 (segment (start 186.666534 76.433466) (end 186.666534 78.229699) (width 0.4) (layer "B.Cu") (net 8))
 (segment (start 187.5 75.6) (end 186.666534 76.433466) (width 0.4) (layer "B.Cu") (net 8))
 (segment (start 208.72675 82.277918) (end 210.7 80.304668) (width 0.4) (layer "B.Cu") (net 8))
 (segment (start 196 75) (end 196 81) (width 0.4) (layer "F.Cu") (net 4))
 (segment (start 196 75) (end 196.1 75.1) (width 0.4) (layer "F.Cu") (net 4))
 (via (at 196 75) (size 1.5) (drill 0.8) (layers "F.Cu" "B.Cu") (free yes) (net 4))
 (via (at 196 81) (size 1.5) (drill 0.8) (layers "F.Cu" "B.Cu") (free yes) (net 4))
 (segment (start 189.882017 76.1) (end 189.781017 76.201) (width 0.4) (layer "B.Cu") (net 4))
 (segment (start 189.9 76.1) (end 189.882017 76.1) (width 0.4) (layer "B.Cu") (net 4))
 (segment (start 192.3 73.7) (end 189.9 76.1) (width 0.4) (layer "B.Cu") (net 4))
 (segment (start 194.7 73.7) (end 192.3 73.7) (width 0.4) (layer "B.Cu") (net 4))
 (segment (start 196 75) (end 194.7 73.7) (width 0.4) (layer "B.Cu") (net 4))
 (segment (start 188.699 76.201) (end 187.936534 76.963466) (width 0.4) (layer "B.Cu") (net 4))
 (segment (start 187.936534 76.963466) (end 187.936534 78.229699) (width 0.4) (layer "B.Cu") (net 4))
 (segment (start 194.843694 83.140178) (end 194.843694 82.156306) (width 0.4) (layer "B.Cu") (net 4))
 (segment (start 194.843694 82.156306) (end 196 81) (width 0.4) (layer "B.Cu") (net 4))
 (segment (start 189.781017 76.201) (end 188.699 76.201) (width 0.4) (layer "B.Cu") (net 4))
 (segment (start 186.455713 73.848811) (end 186.666534 74.059632) (width 0.2) (layer "B.Cu") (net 7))
 (segment (start 181.215969 74.899811) (end 182.366969 73.748811) (width 0.4) (layer "B.Cu") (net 7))
 (segment (start 186.355713 73.748811) (end 186.666534 74.059632) (width 0.4) (layer "B.Cu") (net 7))
 (segment (start 182.366969 73.748811) (end 186.355713 73.748811) (width 0.4) (layer "B.Cu") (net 7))
 (segment (start 196.47676 79.849) (end 198.124173 81.496413) (width 0.4) (layer "B.Cu") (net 5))
 (segment (start 193.731 79.849) (end 196.47676 79.849) (width 0.4) (layer "B.Cu") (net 5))
 (segment (start 198.124173 81.496413) (end 198.124173 83.4) (width 0.4) (layer "B.Cu") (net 5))
 (segment (start 193.6 79.98) (end 193.6 83.113872) (width 0.4) (layer "B.Cu") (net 5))
 (segment (start 193.5 80.08) (end 193.731 79.849) (width 0.4) (layer "B.Cu") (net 5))
 (segment (start 193.6 83.113872) (end 193.573694 83.140178) (width 0.4) (layer "B.Cu") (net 5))
 (segment (start 182.5 78.69578) (end 182.5 80.5) (width 0.4) (layer "B.Cu") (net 6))
 (segment (start 185.311317 81.919811) (end 186.264837 81.919811) (width 0.4) (layer "B.Cu") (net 6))
 (segment (start 185.310317 81.918811) (end 185.311317 81.919811) (width 0.4) (layer "B.Cu") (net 6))
 (segment (start 188.581189 81.918811) (end 192.199 78.301) (width 0.4) (layer "B.Cu") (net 6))
 (segment (start 183.34802 81.3) (end 184.5 81.3) (width 0.4) (layer "B.Cu") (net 6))
 (segment (start 183.755969 77.439811) (end 182.5 78.69578) (width 0.4) (layer "B.Cu") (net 6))
 (segment (start 183.32401 81.32401) (end 183.34802 81.3) (width 0.4) (layer "B.Cu") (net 6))
 (segment (start 184.5 81.3) (end 185.118811 81.918811) (width 0.4) (layer "B.Cu") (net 6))
 (segment (start 186.265837 81.918811) (end 188.581189 81.918811) (width 0.4) (layer "B.Cu") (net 6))
 (segment (start 186.264837 81.919811) (end 186.265837 81.918811) (width 0.4) (layer "B.Cu") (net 6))
 (segment (start 185.118811 81.918811) (end 185.310317 81.918811) (width 0.4) (layer "B.Cu") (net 6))
 (segment (start 182.5 80.5) (end 183.32401 81.32401) (width 0.4) (layer "B.Cu") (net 6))
 (segment (start 192.199 78.301) (end 198.895907 78.301) (width 0.4) (layer "B.Cu") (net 6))
 (segment (start 200.664173 80.069266) (end 200.664173 83.4) (width 0.4) (layer "B.Cu") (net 6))
 (segment (start 198.895907 78.301) (end 200.664173 80.069266) (width 0.4) (layer "B.Cu") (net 6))
 (segment (start 203.870937 77.325421) (end 204.174579 77.325421) (width 1) (layer "B.Cu") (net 9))
 (segment (start 204.174579 77.325421) (end 206.722082 74.777918) (width 1) (layer "B.Cu") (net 9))
 (segment (start 206.722082 74.777918) (end 208.72675 74.777918) (width 1) (layer "B.Cu") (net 9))
 (segment (start 185.039605 83.669811) (end 185.4 83.309416) (width 0.4) (layer "F.Cu") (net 11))
 (segment (start 185.4 81.156888) (end 185.788077 80.768811) (width 0.4) (layer "F.Cu") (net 11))
 (segment (start 185.4 83.309416) (end 185.4 81.156888) (width 0.4) (layer "F.Cu") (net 11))
 (segment (start 185.191532 83.669811) (end 185.039605 83.669811) (width 0.4) (layer "F.Cu") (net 11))
 (via (at 185.788077 80.768811) (size 1.5) (drill 0.8) (layers "F.Cu" "B.Cu") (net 11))
 (via (at 185.191532 83.669811) (size 1.5) (drill 0.8) (layers "F.Cu" "B.Cu") (free yes) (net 11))
 (segment (start 199.144849 77.7) (end 191.813233 77.7) (width 0.4) (layer "B.Cu") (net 11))
 (segment (start 203.839937 82.395088) (end 199.144849 77.7) (width 0.4) (layer "B.Cu") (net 11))
 (segment (start 185 83.9) (end 182.596158 83.9) (width 0.4) (layer "B.Cu") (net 11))
 (segment (start 203.838261 82.95741) (end 203.835025 82.954174) (width 0.4) (layer "B.Cu") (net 11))
 (segment (start 179.8 78.85578) (end 179.8 81.103842) (width 0.4) (layer "B.Cu") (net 11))
 (segment (start 181.215969 77.439811) (end 179.8 78.85578) (width 0.4) (layer "B.Cu") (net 11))
 (segment (start 203.835025 82.954174) (end 203.835025 82.4) (width 0.4) (layer "B.Cu") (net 11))
 (segment (start 188.744422 80.768811) (end 185.788077 80.768811) (width 0.4) (layer "B.Cu") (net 11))
 (segment (start 203.835025 82.4) (end 203.839937 82.395088) (width 0.4) (layer "B.Cu") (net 11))
 (segment (start 182.596158 83.9) (end 181.215969 82.519811) (width 0.4) (layer "B.Cu") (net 11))
 (segment (start 191.813233 77.7) (end 188.744422 80.768811) (width 0.4) (layer "B.Cu") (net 11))
 (segment (start 179.8 81.103842) (end 181.215969 82.519811) (width 0.4) (layer "B.Cu") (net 11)))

